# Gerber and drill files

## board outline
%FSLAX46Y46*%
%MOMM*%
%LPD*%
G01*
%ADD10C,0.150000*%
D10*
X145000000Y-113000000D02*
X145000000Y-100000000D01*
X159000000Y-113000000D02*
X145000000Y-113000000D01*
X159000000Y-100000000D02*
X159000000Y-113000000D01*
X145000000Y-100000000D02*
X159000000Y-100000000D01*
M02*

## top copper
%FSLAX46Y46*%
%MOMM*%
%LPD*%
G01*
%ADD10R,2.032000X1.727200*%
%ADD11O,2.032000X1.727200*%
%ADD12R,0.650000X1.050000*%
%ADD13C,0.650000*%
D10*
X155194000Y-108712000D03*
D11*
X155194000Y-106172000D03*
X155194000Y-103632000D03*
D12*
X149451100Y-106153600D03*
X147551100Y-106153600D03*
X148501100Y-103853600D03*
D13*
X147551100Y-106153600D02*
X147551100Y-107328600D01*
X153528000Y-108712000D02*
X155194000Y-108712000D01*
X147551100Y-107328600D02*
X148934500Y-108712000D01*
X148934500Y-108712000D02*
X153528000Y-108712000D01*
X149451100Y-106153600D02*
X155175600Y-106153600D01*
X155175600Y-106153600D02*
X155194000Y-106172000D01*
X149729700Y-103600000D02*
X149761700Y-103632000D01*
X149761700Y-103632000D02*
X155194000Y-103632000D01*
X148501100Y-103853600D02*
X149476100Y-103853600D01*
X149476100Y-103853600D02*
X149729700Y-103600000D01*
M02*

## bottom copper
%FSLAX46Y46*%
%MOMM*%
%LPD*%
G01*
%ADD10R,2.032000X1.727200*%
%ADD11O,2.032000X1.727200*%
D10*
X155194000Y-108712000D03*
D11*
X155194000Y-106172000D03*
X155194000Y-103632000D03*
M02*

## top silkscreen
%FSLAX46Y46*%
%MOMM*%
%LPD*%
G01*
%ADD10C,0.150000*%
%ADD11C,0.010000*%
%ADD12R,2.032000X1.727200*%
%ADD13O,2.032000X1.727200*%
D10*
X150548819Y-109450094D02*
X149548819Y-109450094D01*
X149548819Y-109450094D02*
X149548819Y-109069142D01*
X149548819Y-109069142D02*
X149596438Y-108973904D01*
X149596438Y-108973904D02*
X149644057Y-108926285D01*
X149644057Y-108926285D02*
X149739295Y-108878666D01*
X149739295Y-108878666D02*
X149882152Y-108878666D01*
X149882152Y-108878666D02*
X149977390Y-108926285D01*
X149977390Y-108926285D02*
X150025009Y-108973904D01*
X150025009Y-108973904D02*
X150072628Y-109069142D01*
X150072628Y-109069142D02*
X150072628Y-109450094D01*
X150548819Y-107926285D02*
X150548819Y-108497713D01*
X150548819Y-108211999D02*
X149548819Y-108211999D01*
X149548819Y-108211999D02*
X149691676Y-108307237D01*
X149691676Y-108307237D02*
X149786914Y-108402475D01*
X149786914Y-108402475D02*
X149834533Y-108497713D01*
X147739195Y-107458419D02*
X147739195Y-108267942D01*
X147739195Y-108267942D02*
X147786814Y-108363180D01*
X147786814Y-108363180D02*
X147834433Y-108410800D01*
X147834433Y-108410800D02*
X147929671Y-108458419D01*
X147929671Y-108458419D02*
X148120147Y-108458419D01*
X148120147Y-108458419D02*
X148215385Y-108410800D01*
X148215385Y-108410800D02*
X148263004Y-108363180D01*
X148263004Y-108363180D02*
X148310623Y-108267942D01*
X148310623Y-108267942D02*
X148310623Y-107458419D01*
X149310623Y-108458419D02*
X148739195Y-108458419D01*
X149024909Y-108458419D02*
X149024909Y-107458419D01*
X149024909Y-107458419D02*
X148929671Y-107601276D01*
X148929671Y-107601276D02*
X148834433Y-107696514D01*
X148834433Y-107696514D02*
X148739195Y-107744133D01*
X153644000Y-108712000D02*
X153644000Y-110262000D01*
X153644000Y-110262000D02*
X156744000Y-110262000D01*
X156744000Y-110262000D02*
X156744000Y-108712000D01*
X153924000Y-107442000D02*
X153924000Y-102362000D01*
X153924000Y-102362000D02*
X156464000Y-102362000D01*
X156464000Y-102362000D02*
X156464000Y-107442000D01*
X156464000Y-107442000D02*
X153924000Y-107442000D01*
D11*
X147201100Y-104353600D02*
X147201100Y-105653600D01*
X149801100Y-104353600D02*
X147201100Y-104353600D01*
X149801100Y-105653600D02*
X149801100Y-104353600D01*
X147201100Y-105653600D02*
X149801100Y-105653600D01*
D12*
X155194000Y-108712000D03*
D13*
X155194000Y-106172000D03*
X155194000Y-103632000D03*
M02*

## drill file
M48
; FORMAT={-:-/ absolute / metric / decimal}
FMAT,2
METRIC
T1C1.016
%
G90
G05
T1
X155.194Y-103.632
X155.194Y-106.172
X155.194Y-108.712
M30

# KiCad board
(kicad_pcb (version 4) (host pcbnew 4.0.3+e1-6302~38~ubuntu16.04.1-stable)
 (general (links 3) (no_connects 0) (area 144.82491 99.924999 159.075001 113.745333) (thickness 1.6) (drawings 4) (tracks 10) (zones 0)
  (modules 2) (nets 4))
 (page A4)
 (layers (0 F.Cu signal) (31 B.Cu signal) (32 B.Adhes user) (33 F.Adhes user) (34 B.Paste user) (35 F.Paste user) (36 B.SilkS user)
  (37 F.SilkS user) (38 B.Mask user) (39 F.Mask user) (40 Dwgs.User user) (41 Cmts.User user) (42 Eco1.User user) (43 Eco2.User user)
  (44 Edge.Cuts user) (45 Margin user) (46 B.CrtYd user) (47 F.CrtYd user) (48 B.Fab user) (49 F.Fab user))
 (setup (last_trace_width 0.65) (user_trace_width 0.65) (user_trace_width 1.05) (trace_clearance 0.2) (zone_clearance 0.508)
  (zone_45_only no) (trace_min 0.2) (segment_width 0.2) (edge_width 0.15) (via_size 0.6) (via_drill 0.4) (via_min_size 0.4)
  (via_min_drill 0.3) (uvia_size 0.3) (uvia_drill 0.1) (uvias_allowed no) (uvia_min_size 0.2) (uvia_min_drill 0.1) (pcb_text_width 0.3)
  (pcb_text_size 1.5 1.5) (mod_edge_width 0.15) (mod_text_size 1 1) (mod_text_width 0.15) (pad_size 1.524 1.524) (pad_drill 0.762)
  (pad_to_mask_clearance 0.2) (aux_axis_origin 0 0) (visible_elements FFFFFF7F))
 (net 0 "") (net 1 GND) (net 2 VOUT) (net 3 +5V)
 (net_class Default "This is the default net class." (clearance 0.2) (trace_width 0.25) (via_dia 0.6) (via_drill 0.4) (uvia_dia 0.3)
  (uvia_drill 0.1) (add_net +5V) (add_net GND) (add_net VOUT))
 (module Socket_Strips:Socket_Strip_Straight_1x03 (layer F.Cu) (at 155.194 108.712 90)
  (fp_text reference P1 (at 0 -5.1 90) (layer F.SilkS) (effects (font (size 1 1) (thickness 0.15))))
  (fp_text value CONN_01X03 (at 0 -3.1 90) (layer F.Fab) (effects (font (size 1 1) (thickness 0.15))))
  (fp_line (start 0 -1.55) (end -1.55 -1.55) (layer F.SilkS) (width 0.15))
  (fp_line (start -1.55 -1.55) (end -1.55 1.55) (layer F.SilkS) (width 0.15))
  (fp_line (start -1.55 1.55) (end 0 1.55) (layer F.SilkS) (width 0.15))
  (fp_line (start 1.27 -1.27) (end 6.35 -1.27) (layer F.SilkS) (width 0.15))
  (fp_line (start 6.35 -1.27) (end 6.35 1.27) (layer F.SilkS) (width 0.15))
  (fp_line (start 6.35 1.27) (end 1.27 1.27) (layer F.SilkS) (width 0.15))
  (fp_line (start 1.27 1.27) (end 1.27 -1.27) (layer F.SilkS) (width 0.15))
  (pad 1 thru_hole rect (at 0 0 90) (size 1.7272 2.032) (drill 1.016) (layers *.Cu *.Mask F.SilkS) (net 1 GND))
  (pad 2 thru_hole oval (at 2.54 0 90) (size 1.7272 2.032) (drill 1.016) (layers *.Cu *.Mask F.SilkS) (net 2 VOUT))
  (pad 3 thru_hole oval (at 5.08 0 90) (size 1.7272 2.032) (drill 1.016) (layers *.Cu *.Mask F.SilkS) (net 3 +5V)))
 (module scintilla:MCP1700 (layer F.Cu) (at 148.5011 105.0036)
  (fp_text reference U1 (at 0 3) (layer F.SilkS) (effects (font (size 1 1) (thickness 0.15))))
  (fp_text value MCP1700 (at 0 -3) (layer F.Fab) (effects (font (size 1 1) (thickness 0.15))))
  (fp_line (start -1.3 -0.65) (end -1.3 0.65) (layer F.SilkS) (width 0.01))
  (fp_line (start 1.3 -0.65) (end -1.3 -0.65) (layer F.SilkS) (width 0.01))
  (fp_line (start 1.3 0.65) (end 1.3 -0.65) (layer F.SilkS) (width 0.01))
  (fp_line (start -1.3 0.65) (end 1.3 0.65) (layer F.SilkS) (width 0.01))
  (pad 2 smd rect (at 0.95 1.15) (size 0.65 1.05) (layers F.Cu F.Paste F.Mask) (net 2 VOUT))
  (pad 1 smd rect (at -0.95 1.15) (size 0.65 1.05) (layers F.Cu F.Paste F.Mask) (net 1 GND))
  (pad 3 smd rect (at 0 -1.15) (size 0.65 1.05) (layers F.Cu F.Paste F.Mask) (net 3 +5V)))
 (gr_line (start 145 113) (end 145 100) (layer Edge.Cuts) (width 0.15))
 (gr_line (start 159 113) (end 145 113) (layer Edge.Cuts) (width 0.15))
 (gr_line (start 159 100) (end 159 113) (layer Edge.Cuts) (width 0.15))
 (gr_line (start 145 100) (end 159 100) (layer Edge.Cuts) (width 0.15))
 (segment (start 147.5511 106.1536) (end 147.5511 107.3286) (width 0.65) (layer F.Cu) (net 1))
 (segment (start 153.528 108.712) (end 155.194 108.712) (width 0.65) (layer F.Cu) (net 1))
 (segment (start 147.5511 107.3286) (end 148.9345 108.712) (width 0.65) (layer F.Cu) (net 1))
 (segment (start 148.9345 108.712) (end 153.528 108.712) (width 0.65) (layer F.Cu) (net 1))
 (segment (start 149.4511 106.1536) (end 155.1756 106.1536) (width 0.65) (layer F.Cu) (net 2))
 (segment (start 155.1756 106.1536) (end 155.194 106.172) (width 0.65) (layer F.Cu) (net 2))
 (segment (start 149.7297 103.6) (end 149.7617 103.632) (width 0.65) (layer F.Cu) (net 3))
 (segment (start 149.7617 103.632) (end 155.194 103.632) (width 0.65) (layer F.Cu) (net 3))
 (segment (start 148.5011 103.8536) (end 149.4761 103.8536) (width 0.65) (layer F.Cu) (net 3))
 (segment (start 149.4761 103.8536) (end 149.7297 103.6) (width 0.65) (layer F.Cu) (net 3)))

